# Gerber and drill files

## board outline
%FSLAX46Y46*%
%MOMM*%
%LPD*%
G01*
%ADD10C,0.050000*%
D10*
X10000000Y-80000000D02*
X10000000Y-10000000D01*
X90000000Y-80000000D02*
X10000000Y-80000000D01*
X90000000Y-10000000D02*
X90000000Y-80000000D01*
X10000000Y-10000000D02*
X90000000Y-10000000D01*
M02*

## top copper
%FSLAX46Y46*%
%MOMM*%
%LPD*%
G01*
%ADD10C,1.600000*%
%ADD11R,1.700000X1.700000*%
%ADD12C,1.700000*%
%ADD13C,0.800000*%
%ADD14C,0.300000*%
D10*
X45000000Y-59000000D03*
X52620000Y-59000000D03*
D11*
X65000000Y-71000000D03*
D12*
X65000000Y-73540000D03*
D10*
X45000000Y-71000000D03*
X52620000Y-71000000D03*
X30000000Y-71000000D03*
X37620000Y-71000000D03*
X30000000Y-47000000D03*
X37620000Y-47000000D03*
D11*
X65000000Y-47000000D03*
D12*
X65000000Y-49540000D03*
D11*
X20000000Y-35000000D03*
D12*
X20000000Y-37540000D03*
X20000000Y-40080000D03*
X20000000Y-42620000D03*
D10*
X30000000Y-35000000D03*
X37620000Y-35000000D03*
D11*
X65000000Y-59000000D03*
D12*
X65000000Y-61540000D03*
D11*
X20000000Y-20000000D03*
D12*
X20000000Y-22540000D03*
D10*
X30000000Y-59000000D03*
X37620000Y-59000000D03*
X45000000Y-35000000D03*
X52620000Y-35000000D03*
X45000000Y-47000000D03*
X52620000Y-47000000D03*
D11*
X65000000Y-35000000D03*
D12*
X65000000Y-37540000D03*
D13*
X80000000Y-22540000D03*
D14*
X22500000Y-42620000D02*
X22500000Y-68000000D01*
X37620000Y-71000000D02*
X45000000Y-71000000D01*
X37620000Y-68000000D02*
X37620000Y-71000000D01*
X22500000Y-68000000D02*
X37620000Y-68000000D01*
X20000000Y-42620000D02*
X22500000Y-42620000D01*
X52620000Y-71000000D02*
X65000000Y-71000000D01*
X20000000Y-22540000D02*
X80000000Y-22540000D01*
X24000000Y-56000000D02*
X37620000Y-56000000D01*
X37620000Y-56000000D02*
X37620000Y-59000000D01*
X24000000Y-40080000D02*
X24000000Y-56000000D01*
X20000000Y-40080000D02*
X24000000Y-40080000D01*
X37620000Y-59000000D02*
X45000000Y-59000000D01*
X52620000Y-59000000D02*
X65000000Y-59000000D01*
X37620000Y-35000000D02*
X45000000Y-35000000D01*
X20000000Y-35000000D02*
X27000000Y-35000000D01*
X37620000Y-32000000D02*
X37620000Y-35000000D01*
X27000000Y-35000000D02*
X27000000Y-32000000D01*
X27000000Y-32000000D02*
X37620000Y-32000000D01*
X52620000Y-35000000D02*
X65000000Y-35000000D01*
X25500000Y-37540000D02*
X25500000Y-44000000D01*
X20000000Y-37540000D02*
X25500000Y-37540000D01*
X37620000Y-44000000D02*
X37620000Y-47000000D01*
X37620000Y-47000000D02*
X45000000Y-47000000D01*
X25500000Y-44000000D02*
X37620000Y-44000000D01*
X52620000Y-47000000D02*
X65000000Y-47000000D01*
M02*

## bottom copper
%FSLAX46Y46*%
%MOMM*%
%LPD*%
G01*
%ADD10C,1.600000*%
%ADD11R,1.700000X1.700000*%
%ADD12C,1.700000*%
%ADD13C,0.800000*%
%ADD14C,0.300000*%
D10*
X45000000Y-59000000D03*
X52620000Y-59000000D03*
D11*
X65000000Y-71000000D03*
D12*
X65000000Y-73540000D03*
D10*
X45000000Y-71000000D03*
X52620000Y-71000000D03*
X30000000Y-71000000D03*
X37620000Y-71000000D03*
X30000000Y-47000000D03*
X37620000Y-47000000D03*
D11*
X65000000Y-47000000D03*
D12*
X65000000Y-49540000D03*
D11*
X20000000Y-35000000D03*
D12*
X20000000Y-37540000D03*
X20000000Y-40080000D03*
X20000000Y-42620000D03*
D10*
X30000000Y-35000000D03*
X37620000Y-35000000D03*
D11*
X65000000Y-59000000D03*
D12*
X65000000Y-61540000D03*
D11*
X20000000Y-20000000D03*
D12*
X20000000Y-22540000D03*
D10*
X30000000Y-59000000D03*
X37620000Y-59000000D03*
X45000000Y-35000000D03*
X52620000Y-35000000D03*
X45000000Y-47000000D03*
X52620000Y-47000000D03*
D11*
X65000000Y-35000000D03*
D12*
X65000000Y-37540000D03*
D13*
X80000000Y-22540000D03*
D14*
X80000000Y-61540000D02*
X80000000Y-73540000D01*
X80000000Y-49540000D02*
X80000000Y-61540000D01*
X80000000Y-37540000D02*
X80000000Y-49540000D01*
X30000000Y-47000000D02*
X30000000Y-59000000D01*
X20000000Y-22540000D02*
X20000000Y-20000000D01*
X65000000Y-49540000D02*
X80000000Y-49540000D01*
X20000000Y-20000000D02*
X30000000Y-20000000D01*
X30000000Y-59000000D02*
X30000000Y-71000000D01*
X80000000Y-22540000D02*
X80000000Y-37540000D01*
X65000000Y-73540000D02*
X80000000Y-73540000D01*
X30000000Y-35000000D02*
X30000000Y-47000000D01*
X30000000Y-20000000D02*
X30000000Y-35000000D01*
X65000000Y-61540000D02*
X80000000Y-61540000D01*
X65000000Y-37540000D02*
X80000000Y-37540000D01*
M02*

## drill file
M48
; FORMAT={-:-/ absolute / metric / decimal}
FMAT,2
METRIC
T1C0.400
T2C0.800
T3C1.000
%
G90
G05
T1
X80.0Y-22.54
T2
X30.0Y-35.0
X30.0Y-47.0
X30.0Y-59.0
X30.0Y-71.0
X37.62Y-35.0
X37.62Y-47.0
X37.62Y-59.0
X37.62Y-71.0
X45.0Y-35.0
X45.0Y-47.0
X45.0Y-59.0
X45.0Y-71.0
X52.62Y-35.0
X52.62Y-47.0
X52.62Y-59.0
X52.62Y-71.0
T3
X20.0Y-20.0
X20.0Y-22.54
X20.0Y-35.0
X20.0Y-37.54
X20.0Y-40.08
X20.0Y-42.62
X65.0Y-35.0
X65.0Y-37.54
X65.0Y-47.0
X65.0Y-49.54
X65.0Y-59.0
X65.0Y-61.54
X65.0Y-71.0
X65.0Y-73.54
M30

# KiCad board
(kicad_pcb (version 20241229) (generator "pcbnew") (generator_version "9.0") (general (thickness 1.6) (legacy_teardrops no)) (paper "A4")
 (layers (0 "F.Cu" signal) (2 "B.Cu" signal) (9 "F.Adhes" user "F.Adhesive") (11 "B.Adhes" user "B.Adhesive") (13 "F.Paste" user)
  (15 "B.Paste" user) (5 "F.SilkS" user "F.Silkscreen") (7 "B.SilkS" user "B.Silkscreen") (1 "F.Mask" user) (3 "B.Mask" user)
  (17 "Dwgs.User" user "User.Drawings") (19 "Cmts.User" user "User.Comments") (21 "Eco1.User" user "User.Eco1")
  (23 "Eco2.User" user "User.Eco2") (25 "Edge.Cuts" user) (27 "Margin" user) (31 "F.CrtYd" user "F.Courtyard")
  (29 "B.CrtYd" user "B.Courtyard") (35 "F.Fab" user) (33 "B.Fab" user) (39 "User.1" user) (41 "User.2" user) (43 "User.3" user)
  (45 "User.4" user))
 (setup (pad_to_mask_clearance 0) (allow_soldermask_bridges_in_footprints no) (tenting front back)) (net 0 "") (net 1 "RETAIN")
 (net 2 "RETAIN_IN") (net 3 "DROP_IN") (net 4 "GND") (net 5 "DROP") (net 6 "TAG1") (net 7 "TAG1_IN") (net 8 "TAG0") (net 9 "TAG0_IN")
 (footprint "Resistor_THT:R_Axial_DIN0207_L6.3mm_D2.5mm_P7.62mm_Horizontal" (layer "F.Cu") (at 45 59)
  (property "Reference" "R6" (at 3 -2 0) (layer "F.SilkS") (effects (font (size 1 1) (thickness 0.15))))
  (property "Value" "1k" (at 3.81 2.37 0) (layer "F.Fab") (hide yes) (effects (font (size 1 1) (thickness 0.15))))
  (pad "1" thru_hole circle (at 0 0) (size 1.6 1.6) (drill 0.8) (layers "*.Cu" "*.Mask") (remove_unused_layers no) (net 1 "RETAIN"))
  (pad "2" thru_hole circle (at 7.62 0) (size 1.6 1.6) (drill 0.8) (layers "*.Cu" "*.Mask") (remove_unused_layers no) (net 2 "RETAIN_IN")))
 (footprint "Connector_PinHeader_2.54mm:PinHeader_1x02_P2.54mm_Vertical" (layer "F.Cu") (at 65 71)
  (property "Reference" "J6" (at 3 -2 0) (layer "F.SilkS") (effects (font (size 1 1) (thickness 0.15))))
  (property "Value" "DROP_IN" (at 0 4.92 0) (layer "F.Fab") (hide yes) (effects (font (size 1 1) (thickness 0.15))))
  (pad "1" thru_hole rect (at 0 0) (size 1.7 1.7) (drill 1) (layers "*.Cu" "*.Mask") (remove_unused_layers no) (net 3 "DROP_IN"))
  (pad "2" thru_hole circle (at 0 2.54) (size 1.7 1.7) (drill 1) (layers "*.Cu" "*.Mask") (remove_unused_layers no) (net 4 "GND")))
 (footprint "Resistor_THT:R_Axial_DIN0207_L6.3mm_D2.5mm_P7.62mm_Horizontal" (layer "F.Cu") (at 45 71)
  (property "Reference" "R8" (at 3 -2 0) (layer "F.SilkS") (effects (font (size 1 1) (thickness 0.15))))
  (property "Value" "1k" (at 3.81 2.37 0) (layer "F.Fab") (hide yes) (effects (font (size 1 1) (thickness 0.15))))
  (pad "1" thru_hole circle (at 0 0) (size 1.6 1.6) (drill 0.8) (layers "*.Cu" "*.Mask") (remove_unused_layers no) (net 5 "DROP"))
  (pad "2" thru_hole circle (at 7.62 0) (size 1.6 1.6) (drill 0.8) (layers "*.Cu" "*.Mask") (remove_unused_layers no) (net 3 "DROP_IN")))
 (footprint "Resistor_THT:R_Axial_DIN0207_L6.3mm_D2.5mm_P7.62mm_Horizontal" (layer "F.Cu") (at 30 71)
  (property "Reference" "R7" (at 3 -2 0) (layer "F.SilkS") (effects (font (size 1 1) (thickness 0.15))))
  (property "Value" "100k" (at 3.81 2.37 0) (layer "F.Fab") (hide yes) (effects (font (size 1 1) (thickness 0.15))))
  (pad "1" thru_hole circle (at 0 0) (size 1.6 1.6) (drill 0.8) (layers "*.Cu" "*.Mask") (remove_unused_layers no) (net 4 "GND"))
  (pad "2" thru_hole circle (at 7.62 0) (size 1.6 1.6) (drill 0.8) (layers "*.Cu" "*.Mask") (remove_unused_layers no) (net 5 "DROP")))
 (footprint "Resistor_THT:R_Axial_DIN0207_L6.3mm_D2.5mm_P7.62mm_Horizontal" (layer "F.Cu") (at 30 47)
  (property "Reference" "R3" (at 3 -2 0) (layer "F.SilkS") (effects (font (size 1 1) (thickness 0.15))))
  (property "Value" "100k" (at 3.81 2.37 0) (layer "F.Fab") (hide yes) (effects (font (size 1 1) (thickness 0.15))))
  (pad "1" thru_hole circle (at 0 0) (size 1.6 1.6) (drill 0.8) (layers "*.Cu" "*.Mask") (remove_unused_layers no) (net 4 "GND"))
  (pad "2" thru_hole circle (at 7.62 0) (size 1.6 1.6) (drill 0.8) (layers "*.Cu" "*.Mask") (remove_unused_layers no) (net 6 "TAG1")))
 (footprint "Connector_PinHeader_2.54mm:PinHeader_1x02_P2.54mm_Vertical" (layer "F.Cu") (at 65 47)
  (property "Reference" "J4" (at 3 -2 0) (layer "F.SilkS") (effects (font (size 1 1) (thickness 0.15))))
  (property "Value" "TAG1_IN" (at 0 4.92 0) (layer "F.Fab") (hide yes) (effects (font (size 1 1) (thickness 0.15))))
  (pad "1" thru_hole rect (at 0 0) (size 1.7 1.7) (drill 1) (layers "*.Cu" "*.Mask") (remove_unused_layers no) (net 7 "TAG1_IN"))
  (pad "2" thru_hole circle (at 0 2.54) (size 1.7 1.7) (drill 1) (layers "*.Cu" "*.Mask") (remove_unused_layers no) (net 4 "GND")))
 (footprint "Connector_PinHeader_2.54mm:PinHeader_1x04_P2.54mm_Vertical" (layer "F.Cu") (at 20 35)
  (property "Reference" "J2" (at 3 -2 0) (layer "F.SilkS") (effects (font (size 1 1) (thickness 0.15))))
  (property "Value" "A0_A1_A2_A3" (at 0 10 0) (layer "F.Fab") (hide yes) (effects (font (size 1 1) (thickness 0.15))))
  (pad "1" thru_hole rect (at 0 0) (size 1.7 1.7) (drill 1) (layers "*.Cu" "*.Mask") (remove_unused_layers no) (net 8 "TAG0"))
  (pad "2" thru_hole circle (at 0 2.54) (size 1.7 1.7) (drill 1) (layers "*.Cu" "*.Mask") (remove_unused_layers no) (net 6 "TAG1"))
  (pad "3" thru_hole circle (at 0 5.08) (size 1.7 1.7) (drill 1) (layers "*.Cu" "*.Mask") (remove_unused_layers no) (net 1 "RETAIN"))
  (pad "4" thru_hole circle (at 0 7.62) (size 1.7 1.7) (drill 1) (layers "*.Cu" "*.Mask") (remove_unused_layers no) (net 5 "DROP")))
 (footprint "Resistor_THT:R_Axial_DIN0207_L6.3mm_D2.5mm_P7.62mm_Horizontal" (layer "F.Cu") (at 30 35)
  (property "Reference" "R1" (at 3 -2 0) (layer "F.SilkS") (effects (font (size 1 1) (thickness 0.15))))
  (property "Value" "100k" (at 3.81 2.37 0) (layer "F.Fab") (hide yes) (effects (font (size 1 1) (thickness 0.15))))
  (pad "1" thru_hole circle (at 0 0) (size 1.6 1.6) (drill 0.8) (layers "*.Cu" "*.Mask") (remove_unused_layers no) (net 4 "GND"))
  (pad "2" thru_hole circle (at 7.62 0) (size 1.6 1.6) (drill 0.8) (layers "*.Cu" "*.Mask") (remove_unused_layers no) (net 8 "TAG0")))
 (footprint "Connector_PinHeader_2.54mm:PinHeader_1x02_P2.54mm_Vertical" (layer "F.Cu") (at 65 59)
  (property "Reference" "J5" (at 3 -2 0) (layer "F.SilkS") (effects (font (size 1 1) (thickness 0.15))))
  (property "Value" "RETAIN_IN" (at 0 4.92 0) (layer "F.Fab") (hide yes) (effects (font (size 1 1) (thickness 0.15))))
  (pad "1" thru_hole rect (at 0 0) (size 1.7 1.7) (drill 1) (layers "*.Cu" "*.Mask") (remove_unused_layers no) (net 2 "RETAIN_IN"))
  (pad "2" thru_hole circle (at 0 2.54) (size 1.7 1.7) (drill 1) (layers "*.Cu" "*.Mask") (remove_unused_layers no) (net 4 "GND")))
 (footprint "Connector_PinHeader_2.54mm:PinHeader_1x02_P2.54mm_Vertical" (layer "F.Cu") (at 20 20)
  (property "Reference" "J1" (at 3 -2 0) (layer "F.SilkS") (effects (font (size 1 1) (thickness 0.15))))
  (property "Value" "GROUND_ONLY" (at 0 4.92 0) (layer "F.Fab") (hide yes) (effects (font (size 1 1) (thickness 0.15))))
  (pad "1" thru_hole rect (at 0 0) (size 1.7 1.7) (drill 1) (layers "*.Cu" "*.Mask") (remove_unused_layers no) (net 4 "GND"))
  (pad "2" thru_hole circle (at 0 2.54) (size 1.7 1.7) (drill 1) (layers "*.Cu" "*.Mask") (remove_unused_layers no) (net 4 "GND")))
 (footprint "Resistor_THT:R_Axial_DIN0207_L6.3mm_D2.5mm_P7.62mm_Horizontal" (layer "F.Cu") (at 30 59)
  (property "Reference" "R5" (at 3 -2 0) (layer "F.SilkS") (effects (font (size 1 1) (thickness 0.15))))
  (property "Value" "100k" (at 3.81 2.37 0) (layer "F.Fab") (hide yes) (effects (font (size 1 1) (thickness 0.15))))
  (pad "1" thru_hole circle (at 0 0) (size 1.6 1.6) (drill 0.8) (layers "*.Cu" "*.Mask") (remove_unused_layers no) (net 4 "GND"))
  (pad "2" thru_hole circle (at 7.62 0) (size 1.6 1.6) (drill 0.8) (layers "*.Cu" "*.Mask") (remove_unused_layers no) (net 1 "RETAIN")))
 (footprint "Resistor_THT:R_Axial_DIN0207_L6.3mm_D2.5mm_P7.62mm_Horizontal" (layer "F.Cu") (at 45 35)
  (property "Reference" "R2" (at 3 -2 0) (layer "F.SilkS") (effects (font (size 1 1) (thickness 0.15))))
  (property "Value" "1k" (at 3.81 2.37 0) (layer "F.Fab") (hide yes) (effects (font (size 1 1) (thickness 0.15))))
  (pad "1" thru_hole circle (at 0 0) (size 1.6 1.6) (drill 0.8) (layers "*.Cu" "*.Mask") (remove_unused_layers no) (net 8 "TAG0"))
  (pad "2" thru_hole circle (at 7.62 0) (size 1.6 1.6) (drill 0.8) (layers "*.Cu" "*.Mask") (remove_unused_layers no) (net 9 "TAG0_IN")))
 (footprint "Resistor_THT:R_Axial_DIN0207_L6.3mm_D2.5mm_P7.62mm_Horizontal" (layer "F.Cu") (at 45 47)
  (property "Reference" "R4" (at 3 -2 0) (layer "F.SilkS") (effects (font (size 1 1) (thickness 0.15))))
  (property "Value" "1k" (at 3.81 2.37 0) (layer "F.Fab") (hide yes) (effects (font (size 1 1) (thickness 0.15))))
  (pad "1" thru_hole circle (at 0 0) (size 1.6 1.6) (drill 0.8) (layers "*.Cu" "*.Mask") (remove_unused_layers no) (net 6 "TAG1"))
  (pad "2" thru_hole circle (at 7.62 0) (size 1.6 1.6) (drill 0.8) (layers "*.Cu" "*.Mask") (remove_unused_layers no) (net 7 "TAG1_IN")))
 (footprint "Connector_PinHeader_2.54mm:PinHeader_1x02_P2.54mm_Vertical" (layer "F.Cu") (at 65 35)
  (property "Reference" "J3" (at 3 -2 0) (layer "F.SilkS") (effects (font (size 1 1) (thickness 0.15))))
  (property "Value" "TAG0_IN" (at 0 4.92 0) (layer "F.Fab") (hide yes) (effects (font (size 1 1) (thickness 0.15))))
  (pad "1" thru_hole rect (at 0 0) (size 1.7 1.7) (drill 1) (layers "*.Cu" "*.Mask") (remove_unused_layers no) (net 9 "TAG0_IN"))
  (pad "2" thru_hole circle (at 0 2.54) (size 1.7 1.7) (drill 1) (layers "*.Cu" "*.Mask") (remove_unused_layers no) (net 4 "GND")))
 (gr_line (start 10 80) (end 10 10) (stroke (width 0.05) (type default)) (layer "Edge.Cuts"))
 (gr_line (start 90 80) (end 10 80) (stroke (width 0.05) (type default)) (layer "Edge.Cuts"))
 (gr_line (start 90 10) (end 90 80) (stroke (width 0.05) (type default)) (layer "Edge.Cuts"))
 (gr_line (start 10 10) (end 90 10) (stroke (width 0.05) (type default)) (layer "Edge.Cuts"))
 (segment (start 22.5 42.62) (end 22.5 68) (width 0.3) (layer "F.Cu") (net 5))
 (segment (start 37.62 71) (end 45 71) (width 0.3) (layer "F.Cu") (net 5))
 (segment (start 37.62 68) (end 37.62 71) (width 0.3) (layer "F.Cu") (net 5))
 (segment (start 22.5 68) (end 37.62 68) (width 0.3) (layer "F.Cu") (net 5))
 (segment (start 20 42.62) (end 22.5 42.62) (width 0.3) (layer "F.Cu") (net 5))
 (segment (start 52.62 71) (end 65 71) (width 0.3) (layer "F.Cu") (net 3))
 (segment (start 20 22.54) (end 80 22.54) (width 0.3) (layer "F.Cu") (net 4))
 (via (at 80 22.54) (size 0.8) (drill 0.4) (layers "F.Cu" "B.Cu") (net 4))
 (segment (start 80 61.54) (end 80 73.54) (width 0.3) (layer "B.Cu") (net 4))
 (segment (start 80 49.54) (end 80 61.54) (width 0.3) (layer "B.Cu") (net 4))
 (segment (start 80 37.54) (end 80 49.54) (width 0.3) (layer "B.Cu") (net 4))
 (segment (start 30 47) (end 30 59) (width 0.3) (layer "B.Cu") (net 4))
 (segment (start 20 22.54) (end 20 20) (width 0.3) (layer "B.Cu") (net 4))
 (segment (start 65 49.54) (end 80 49.54) (width 0.3) (layer "B.Cu") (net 4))
 (segment (start 20 20) (end 30 20) (width 0.3) (layer "B.Cu") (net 4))
 (segment (start 30 59) (end 30 71) (width 0.3) (layer "B.Cu") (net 4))
 (segment (start 80 22.54) (end 80 37.54) (width 0.3) (layer "B.Cu") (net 4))
 (segment (start 65 73.54) (end 80 73.54) (width 0.3) (layer "B.Cu") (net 4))
 (segment (start 30 35) (end 30 47) (width 0.3) (layer "B.Cu") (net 4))
 (segment (start 30 20) (end 30 35) (width 0.3) (layer "B.Cu") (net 4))
 (segment (start 65 61.54) (end 80 61.54) (width 0.3) (layer "B.Cu") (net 4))
 (segment (start 65 37.54) (end 80 37.54) (width 0.3) (layer "B.Cu") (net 4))
 (segment (start 24 56) (end 37.62 56) (width 0.3) (layer "F.Cu") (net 1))
 (segment (start 37.62 56) (end 37.62 59) (width 0.3) (layer "F.Cu") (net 1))
 (segment (start 24 40.08) (end 24 56) (width 0.3) (layer "F.Cu") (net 1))
 (segment (start 20 40.08) (end 24 40.08) (width 0.3) (layer "F.Cu") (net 1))
 (segment (start 37.62 59) (end 45 59) (width 0.3) (layer "F.Cu") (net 1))
 (segment (start 52.62 59) (end 65 59) (width 0.3) (layer "F.Cu") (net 2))
 (segment (start 37.62 35) (end 45 35) (width 0.3) (layer "F.Cu") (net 8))
 (segment (start 20 35) (end 27 35) (width 0.3) (layer "F.Cu") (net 8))
 (segment (start 37.62 32) (end 37.62 35) (width 0.3) (layer "F.Cu") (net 8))
 (segment (start 27 35) (end 27 32) (width 0.3) (layer "F.Cu") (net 8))
 (segment (start 27 32) (end 37.62 32) (width 0.3) (layer "F.Cu") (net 8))
 (segment (start 52.62 35) (end 65 35) (width 0.3) (layer "F.Cu") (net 9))
 (segment (start 25.5 37.54) (end 25.5 44) (width 0.3) (layer "F.Cu") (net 6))
 (segment (start 20 37.54) (end 25.5 37.54) (width 0.3) (layer "F.Cu") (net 6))
 (segment (start 37.62 44) (end 37.62 47) (width 0.3) (layer "F.Cu") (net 6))
 (segment (start 37.62 47) (end 45 47) (width 0.3) (layer "F.Cu") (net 6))
 (segment (start 25.5 44) (end 37.62 44) (width 0.3) (layer "F.Cu") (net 6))
 (segment (start 52.62 47) (end 65 47) (width 0.3) (layer "F.Cu") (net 7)))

